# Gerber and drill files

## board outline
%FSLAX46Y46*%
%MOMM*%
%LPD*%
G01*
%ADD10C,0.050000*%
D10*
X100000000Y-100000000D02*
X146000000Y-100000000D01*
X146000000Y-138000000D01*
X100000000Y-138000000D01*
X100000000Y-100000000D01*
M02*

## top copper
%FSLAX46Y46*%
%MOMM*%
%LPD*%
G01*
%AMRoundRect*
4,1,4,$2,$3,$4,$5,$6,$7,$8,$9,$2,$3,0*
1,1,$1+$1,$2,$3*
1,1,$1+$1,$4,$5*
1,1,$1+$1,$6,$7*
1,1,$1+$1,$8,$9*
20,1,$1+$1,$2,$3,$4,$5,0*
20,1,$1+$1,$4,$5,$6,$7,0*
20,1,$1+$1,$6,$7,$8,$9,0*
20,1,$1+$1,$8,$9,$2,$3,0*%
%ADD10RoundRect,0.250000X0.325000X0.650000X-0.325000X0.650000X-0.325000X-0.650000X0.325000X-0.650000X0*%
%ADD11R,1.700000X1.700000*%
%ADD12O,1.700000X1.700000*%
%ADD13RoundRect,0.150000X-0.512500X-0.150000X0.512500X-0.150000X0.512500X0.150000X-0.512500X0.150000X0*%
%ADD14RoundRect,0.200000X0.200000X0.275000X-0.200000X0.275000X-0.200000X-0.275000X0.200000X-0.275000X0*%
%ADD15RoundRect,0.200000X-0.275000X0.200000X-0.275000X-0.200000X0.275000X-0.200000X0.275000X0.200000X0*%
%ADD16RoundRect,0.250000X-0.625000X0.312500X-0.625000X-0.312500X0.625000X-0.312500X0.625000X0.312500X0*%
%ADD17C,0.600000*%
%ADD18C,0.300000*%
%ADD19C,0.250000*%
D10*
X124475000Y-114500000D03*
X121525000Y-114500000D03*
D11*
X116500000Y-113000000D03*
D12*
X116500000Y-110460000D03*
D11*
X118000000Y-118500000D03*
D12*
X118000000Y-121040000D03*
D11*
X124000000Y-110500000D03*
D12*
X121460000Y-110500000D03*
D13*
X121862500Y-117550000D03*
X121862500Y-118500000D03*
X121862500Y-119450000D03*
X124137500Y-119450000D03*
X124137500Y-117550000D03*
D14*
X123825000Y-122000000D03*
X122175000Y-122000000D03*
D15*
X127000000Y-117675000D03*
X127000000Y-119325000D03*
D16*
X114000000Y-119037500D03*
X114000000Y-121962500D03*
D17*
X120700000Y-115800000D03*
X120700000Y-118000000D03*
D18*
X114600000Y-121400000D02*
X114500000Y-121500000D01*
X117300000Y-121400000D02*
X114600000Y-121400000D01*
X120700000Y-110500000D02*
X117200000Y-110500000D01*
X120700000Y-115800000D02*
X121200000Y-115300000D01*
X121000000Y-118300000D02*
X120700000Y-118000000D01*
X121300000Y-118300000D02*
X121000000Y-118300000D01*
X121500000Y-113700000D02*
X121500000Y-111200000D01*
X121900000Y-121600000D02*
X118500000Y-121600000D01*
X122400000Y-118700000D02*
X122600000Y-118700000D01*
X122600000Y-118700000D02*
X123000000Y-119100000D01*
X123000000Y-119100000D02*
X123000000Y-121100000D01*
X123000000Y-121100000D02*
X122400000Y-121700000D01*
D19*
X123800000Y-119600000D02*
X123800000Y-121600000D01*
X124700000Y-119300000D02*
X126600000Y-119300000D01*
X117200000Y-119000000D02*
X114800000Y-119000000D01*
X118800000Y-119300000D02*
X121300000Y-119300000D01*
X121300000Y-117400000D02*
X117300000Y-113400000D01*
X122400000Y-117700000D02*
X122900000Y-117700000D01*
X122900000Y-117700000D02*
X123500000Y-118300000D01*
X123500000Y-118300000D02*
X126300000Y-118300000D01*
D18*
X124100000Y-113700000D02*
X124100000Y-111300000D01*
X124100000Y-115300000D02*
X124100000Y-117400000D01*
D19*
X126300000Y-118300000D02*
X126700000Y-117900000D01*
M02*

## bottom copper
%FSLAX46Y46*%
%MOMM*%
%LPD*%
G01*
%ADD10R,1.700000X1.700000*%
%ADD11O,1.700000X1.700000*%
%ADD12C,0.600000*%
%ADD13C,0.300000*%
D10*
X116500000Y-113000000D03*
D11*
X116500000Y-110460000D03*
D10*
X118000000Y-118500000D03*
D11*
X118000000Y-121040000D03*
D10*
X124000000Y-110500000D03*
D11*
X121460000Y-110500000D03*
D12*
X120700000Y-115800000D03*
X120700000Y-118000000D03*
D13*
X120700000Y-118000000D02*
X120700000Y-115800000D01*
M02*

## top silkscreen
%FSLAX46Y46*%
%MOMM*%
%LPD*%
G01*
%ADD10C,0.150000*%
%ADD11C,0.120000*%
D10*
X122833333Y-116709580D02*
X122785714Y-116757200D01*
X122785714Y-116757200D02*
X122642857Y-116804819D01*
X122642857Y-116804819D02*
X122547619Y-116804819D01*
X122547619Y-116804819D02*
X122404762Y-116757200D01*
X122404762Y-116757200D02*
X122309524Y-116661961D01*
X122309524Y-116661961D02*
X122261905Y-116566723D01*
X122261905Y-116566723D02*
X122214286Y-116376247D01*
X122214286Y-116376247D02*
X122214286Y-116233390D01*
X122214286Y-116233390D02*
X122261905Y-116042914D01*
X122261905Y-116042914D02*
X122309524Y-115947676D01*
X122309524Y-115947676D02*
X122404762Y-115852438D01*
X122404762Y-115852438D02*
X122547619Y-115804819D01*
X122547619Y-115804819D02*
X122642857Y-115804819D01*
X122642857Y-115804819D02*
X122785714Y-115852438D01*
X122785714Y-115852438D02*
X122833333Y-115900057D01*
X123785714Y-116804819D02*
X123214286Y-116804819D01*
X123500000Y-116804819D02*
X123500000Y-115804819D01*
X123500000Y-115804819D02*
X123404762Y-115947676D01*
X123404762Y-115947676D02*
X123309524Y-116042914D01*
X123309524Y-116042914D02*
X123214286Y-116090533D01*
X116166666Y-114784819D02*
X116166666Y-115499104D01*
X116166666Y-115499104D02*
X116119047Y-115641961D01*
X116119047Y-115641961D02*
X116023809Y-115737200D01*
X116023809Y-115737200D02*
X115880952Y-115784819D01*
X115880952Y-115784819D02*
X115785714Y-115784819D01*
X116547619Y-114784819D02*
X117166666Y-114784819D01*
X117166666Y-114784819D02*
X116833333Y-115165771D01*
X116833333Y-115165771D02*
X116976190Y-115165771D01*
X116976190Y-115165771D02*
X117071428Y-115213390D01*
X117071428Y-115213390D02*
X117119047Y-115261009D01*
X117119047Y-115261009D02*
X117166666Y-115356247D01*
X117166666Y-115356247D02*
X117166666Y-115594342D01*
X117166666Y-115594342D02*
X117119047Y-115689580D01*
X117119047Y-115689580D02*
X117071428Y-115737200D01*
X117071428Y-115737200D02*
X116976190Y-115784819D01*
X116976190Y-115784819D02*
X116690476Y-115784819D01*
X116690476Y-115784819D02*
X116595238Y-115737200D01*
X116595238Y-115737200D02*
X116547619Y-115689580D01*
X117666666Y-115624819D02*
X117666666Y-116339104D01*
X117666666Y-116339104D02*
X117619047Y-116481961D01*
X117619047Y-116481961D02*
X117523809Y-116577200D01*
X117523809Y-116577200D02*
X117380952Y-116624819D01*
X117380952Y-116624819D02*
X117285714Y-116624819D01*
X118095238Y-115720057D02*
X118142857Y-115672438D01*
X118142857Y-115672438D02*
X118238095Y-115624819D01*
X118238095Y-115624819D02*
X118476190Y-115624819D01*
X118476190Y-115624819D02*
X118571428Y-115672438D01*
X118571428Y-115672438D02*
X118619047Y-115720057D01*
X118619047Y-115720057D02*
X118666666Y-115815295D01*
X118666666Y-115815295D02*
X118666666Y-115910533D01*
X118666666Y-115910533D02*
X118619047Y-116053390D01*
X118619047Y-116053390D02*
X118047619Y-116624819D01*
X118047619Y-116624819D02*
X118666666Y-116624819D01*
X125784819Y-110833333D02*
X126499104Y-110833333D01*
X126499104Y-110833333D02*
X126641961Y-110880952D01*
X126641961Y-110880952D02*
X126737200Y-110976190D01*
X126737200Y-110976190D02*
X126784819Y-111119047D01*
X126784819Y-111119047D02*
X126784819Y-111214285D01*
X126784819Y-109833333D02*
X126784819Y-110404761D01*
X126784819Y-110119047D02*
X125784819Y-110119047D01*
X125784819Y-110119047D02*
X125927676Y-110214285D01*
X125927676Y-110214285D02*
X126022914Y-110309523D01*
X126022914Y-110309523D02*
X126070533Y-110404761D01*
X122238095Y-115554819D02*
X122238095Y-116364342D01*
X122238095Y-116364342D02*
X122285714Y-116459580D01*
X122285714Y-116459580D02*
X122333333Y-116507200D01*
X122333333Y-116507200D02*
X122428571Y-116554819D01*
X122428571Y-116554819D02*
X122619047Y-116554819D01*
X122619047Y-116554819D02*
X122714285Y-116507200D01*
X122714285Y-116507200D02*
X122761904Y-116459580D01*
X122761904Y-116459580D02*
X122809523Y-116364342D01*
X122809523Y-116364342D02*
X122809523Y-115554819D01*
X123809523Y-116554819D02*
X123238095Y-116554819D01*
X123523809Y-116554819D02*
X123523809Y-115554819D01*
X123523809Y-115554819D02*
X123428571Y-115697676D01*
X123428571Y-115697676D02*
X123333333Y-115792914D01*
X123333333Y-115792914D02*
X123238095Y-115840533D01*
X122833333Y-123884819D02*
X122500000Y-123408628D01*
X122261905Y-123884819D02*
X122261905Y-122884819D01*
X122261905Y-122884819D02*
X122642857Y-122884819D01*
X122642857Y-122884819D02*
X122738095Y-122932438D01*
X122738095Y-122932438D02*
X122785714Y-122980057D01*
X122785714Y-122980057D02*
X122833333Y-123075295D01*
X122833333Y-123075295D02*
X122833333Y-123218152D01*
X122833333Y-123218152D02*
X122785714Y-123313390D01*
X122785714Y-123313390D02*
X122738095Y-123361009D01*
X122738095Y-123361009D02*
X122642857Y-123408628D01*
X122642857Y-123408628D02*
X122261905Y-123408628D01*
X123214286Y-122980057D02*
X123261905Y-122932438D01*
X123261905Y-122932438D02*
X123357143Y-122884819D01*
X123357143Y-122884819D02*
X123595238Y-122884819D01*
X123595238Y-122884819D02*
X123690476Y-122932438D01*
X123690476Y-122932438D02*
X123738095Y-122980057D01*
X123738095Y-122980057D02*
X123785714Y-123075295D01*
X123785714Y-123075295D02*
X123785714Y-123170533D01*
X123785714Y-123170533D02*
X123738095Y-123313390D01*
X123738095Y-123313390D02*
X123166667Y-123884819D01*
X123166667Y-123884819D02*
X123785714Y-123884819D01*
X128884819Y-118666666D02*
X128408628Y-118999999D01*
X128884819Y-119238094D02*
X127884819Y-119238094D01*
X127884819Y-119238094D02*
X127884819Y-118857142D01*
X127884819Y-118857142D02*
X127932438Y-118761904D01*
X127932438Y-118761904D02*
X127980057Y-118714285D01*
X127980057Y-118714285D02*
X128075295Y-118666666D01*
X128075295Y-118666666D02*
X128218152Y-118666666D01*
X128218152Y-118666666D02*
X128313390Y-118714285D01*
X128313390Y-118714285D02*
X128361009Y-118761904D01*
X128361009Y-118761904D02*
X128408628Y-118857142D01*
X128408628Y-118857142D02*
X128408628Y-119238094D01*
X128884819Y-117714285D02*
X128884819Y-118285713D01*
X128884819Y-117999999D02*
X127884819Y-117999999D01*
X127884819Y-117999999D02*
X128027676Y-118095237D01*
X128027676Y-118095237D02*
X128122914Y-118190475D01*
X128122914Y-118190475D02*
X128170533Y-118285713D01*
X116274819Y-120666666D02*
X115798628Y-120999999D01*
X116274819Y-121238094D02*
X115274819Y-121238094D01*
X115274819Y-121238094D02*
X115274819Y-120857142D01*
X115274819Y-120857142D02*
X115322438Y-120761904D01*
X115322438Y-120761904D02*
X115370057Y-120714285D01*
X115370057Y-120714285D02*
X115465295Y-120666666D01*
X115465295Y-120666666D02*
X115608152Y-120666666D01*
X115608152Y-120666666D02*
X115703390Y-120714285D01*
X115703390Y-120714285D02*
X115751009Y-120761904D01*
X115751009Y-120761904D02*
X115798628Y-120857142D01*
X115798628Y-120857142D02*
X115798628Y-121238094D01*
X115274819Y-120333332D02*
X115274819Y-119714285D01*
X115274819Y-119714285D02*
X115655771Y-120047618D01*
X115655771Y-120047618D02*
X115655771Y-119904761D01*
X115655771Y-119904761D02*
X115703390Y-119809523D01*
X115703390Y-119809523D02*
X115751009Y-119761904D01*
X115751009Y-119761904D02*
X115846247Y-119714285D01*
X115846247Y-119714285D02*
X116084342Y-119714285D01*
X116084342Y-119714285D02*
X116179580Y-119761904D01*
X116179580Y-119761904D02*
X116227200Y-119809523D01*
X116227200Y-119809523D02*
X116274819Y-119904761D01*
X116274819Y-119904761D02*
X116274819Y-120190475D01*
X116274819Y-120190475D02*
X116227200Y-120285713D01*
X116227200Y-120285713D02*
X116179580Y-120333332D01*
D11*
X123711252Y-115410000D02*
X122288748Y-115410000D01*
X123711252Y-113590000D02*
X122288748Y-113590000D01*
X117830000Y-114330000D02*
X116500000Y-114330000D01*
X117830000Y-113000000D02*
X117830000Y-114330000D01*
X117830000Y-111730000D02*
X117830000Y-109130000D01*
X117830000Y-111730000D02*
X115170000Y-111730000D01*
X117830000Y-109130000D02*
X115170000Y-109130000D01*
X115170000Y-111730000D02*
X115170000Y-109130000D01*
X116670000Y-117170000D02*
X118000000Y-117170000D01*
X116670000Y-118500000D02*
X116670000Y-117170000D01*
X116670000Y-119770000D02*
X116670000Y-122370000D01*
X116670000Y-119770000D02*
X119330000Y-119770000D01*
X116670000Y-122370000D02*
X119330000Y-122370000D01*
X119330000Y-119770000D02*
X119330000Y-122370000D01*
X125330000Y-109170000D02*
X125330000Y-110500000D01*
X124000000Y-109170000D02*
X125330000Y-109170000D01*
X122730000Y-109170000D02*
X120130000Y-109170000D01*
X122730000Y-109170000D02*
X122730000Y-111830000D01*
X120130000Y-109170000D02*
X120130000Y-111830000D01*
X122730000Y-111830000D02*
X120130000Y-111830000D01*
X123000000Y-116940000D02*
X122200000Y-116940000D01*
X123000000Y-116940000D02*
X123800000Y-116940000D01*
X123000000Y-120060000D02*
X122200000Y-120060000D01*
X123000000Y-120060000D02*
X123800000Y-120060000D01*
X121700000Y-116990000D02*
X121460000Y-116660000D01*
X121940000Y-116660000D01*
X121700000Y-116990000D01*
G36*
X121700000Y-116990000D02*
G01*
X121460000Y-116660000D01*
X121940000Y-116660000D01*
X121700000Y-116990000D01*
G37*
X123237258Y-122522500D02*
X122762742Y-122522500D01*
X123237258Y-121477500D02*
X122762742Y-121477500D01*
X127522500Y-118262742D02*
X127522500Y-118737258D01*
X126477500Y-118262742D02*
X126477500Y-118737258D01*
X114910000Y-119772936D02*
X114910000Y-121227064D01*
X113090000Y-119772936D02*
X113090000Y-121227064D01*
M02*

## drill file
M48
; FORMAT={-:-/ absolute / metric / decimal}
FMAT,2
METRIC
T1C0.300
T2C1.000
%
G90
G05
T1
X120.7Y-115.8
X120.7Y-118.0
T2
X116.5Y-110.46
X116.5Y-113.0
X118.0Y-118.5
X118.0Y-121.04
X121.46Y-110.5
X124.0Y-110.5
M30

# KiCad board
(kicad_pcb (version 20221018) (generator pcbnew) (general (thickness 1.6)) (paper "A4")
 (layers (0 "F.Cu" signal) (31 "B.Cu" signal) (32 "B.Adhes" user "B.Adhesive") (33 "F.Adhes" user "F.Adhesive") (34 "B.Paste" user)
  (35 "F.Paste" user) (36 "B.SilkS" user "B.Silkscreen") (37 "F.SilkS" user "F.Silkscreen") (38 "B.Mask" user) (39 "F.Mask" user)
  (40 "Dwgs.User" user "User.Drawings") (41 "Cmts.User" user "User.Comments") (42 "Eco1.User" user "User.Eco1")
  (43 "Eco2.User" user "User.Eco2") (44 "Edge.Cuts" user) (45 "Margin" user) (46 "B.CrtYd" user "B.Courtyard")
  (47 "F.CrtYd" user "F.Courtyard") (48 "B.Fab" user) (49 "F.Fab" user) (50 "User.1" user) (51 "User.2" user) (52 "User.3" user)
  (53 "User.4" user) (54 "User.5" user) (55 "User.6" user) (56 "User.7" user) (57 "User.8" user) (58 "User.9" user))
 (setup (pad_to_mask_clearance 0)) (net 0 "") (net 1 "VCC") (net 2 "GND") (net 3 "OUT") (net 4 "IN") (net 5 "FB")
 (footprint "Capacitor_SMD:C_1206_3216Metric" (layer "F.Cu") (at 123 114.5 180)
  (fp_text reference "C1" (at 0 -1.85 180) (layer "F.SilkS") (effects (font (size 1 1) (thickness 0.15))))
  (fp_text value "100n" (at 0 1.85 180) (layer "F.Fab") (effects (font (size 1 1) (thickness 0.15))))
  (fp_line (start -0.711252 -0.91) (end 0.711252 -0.91) (stroke (width 0.12) (type solid)) (layer "F.SilkS"))
  (fp_line (start -0.711252 0.91) (end 0.711252 0.91) (stroke (width 0.12) (type solid)) (layer "F.SilkS"))
  (pad "1" smd roundrect (at -1.475 0 180) (size 1.15 1.8) (layers "F.Cu" "F.Paste" "F.Mask") (roundrect_rratio 0.217391) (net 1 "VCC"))
  (pad "2" smd roundrect (at 1.475 0 180) (size 1.15 1.8) (layers "F.Cu" "F.Paste" "F.Mask") (roundrect_rratio 0.217391) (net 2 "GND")))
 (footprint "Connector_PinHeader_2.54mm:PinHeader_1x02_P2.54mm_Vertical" (layer "F.Cu") (at 116.5 113 180)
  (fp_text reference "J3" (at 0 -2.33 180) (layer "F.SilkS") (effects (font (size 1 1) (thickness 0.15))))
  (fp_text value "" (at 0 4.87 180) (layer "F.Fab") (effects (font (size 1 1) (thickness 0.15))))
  (fp_line (start -1.33 -1.33) (end 0 -1.33) (stroke (width 0.12) (type solid)) (layer "F.SilkS"))
  (fp_line (start -1.33 0) (end -1.33 -1.33) (stroke (width 0.12) (type solid)) (layer "F.SilkS"))
  (fp_line (start -1.33 1.27) (end -1.33 3.87) (stroke (width 0.12) (type solid)) (layer "F.SilkS"))
  (fp_line (start -1.33 1.27) (end 1.33 1.27) (stroke (width 0.12) (type solid)) (layer "F.SilkS"))
  (fp_line (start -1.33 3.87) (end 1.33 3.87) (stroke (width 0.12) (type solid)) (layer "F.SilkS"))
  (fp_line (start 1.33 1.27) (end 1.33 3.87) (stroke (width 0.12) (type solid)) (layer "F.SilkS"))
  (pad "1" thru_hole rect (at 0 0 180) (size 1.7 1.7) (drill 1) (layers "*.Cu" "*.Mask") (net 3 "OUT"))
  (pad "2" thru_hole oval (at 0 2.54 180) (size 1.7 1.7) (drill 1) (layers "*.Cu" "*.Mask") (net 2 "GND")))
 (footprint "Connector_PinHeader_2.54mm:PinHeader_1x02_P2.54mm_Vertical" (layer "F.Cu") (at 118 118.5)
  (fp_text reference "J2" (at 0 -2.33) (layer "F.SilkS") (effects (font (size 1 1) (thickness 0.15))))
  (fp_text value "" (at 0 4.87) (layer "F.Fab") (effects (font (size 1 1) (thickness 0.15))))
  (fp_line (start -1.33 -1.33) (end 0 -1.33) (stroke (width 0.12) (type solid)) (layer "F.SilkS"))
  (fp_line (start -1.33 0) (end -1.33 -1.33) (stroke (width 0.12) (type solid)) (layer "F.SilkS"))
  (fp_line (start -1.33 1.27) (end -1.33 3.87) (stroke (width 0.12) (type solid)) (layer "F.SilkS"))
  (fp_line (start -1.33 1.27) (end 1.33 1.27) (stroke (width 0.12) (type solid)) (layer "F.SilkS"))
  (fp_line (start -1.33 3.87) (end 1.33 3.87) (stroke (width 0.12) (type solid)) (layer "F.SilkS"))
  (fp_line (start 1.33 1.27) (end 1.33 3.87) (stroke (width 0.12) (type solid)) (layer "F.SilkS"))
  (pad "1" thru_hole rect (at 0 0) (size 1.7 1.7) (drill 1) (layers "*.Cu" "*.Mask") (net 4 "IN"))
  (pad "2" thru_hole oval (at 0 2.54) (size 1.7 1.7) (drill 1) (layers "*.Cu" "*.Mask") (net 2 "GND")))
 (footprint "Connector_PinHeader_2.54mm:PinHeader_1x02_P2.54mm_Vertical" (layer "F.Cu") (at 124 110.5 -90)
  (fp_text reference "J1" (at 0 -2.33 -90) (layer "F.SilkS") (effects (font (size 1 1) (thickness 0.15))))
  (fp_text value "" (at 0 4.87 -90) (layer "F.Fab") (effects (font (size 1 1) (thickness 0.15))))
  (fp_line (start -1.33 -1.33) (end 0 -1.33) (stroke (width 0.12) (type solid)) (layer "F.SilkS"))
  (fp_line (start -1.33 0) (end -1.33 -1.33) (stroke (width 0.12) (type solid)) (layer "F.SilkS"))
  (fp_line (start -1.33 1.27) (end -1.33 3.87) (stroke (width 0.12) (type solid)) (layer "F.SilkS"))
  (fp_line (start -1.33 1.27) (end 1.33 1.27) (stroke (width 0.12) (type solid)) (layer "F.SilkS"))
  (fp_line (start -1.33 3.87) (end 1.33 3.87) (stroke (width 0.12) (type solid)) (layer "F.SilkS"))
  (fp_line (start 1.33 1.27) (end 1.33 3.87) (stroke (width 0.12) (type solid)) (layer "F.SilkS"))
  (pad "1" thru_hole rect (at 0 0 270) (size 1.7 1.7) (drill 1) (layers "*.Cu" "*.Mask") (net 1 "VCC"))
  (pad "2" thru_hole oval (at 0 2.54 270) (size 1.7 1.7) (drill 1) (layers "*.Cu" "*.Mask") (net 2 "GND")))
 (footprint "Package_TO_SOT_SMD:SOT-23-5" (layer "F.Cu") (at 123 118.5)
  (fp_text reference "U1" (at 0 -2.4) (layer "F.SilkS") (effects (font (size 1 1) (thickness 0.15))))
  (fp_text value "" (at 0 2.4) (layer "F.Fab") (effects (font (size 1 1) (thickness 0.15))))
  (fp_line (start 0 -1.56) (end -0.8 -1.56) (stroke (width 0.12) (type solid)) (layer "F.SilkS"))
  (fp_line (start 0 -1.56) (end 0.8 -1.56) (stroke (width 0.12) (type solid)) (layer "F.SilkS"))
  (fp_line (start 0 1.56) (end -0.8 1.56) (stroke (width 0.12) (type solid)) (layer "F.SilkS"))
  (fp_line (start 0 1.56) (end 0.8 1.56) (stroke (width 0.12) (type solid)) (layer "F.SilkS"))
  (fp_poly
   (pts (xy -1.3 -1.51) (xy -1.54 -1.84) (xy -1.06 -1.84) (xy -1.3 -1.51)) (stroke (width 0.12) (type solid)) (fill solid) (layer "F.SilkS"))
  (pad "1" smd roundrect (at -1.1375 -0.95) (size 1.325 0.6) (layers "F.Cu" "F.Paste" "F.Mask") (roundrect_rratio 0.25) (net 3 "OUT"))
  (pad "2" smd roundrect (at -1.1375 0) (size 1.325 0.6) (layers "F.Cu" "F.Paste" "F.Mask") (roundrect_rratio 0.25) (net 2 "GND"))
  (pad "3" smd roundrect (at -1.1375 0.95) (size 1.325 0.6) (layers "F.Cu" "F.Paste" "F.Mask") (roundrect_rratio 0.25) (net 4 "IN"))
  (pad "4" smd roundrect (at 1.1375 0.95) (size 1.325 0.6) (layers "F.Cu" "F.Paste" "F.Mask") (roundrect_rratio 0.25) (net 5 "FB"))
  (pad "5" smd roundrect (at 1.1375 -0.95) (size 1.325 0.6) (layers "F.Cu" "F.Paste" "F.Mask") (roundrect_rratio 0.25) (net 1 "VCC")))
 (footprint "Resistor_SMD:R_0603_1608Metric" (layer "F.Cu") (at 123 122 180)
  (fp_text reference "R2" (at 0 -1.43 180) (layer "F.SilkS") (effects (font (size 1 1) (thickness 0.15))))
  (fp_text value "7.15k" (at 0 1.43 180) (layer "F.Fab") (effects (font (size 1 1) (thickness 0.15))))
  (fp_line (start -0.237258 -0.5225) (end 0.237258 -0.5225) (stroke (width 0.12) (type solid)) (layer "F.SilkS"))
  (fp_line (start -0.237258 0.5225) (end 0.237258 0.5225) (stroke (width 0.12) (type solid)) (layer "F.SilkS"))
  (pad "1" smd roundrect (at -0.825 0 180) (size 0.8 0.95) (layers "F.Cu" "F.Paste" "F.Mask") (roundrect_rratio 0.25) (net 5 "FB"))
  (pad "2" smd roundrect (at 0.825 0 180) (size 0.8 0.95) (layers "F.Cu" "F.Paste" "F.Mask") (roundrect_rratio 0.25) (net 2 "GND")))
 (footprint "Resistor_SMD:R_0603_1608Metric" (layer "F.Cu") (at 127 118.5 -90)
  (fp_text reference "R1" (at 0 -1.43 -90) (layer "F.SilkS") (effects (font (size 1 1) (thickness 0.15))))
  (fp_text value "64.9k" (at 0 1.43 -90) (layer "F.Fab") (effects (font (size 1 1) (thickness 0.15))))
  (fp_line (start -0.237258 -0.5225) (end 0.237258 -0.5225) (stroke (width 0.12) (type solid)) (layer "F.SilkS"))
  (fp_line (start -0.237258 0.5225) (end 0.237258 0.5225) (stroke (width 0.12) (type solid)) (layer "F.SilkS"))
  (pad "1" smd roundrect (at -0.825 0 270) (size 0.8 0.95) (layers "F.Cu" "F.Paste" "F.Mask") (roundrect_rratio 0.25) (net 3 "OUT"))
  (pad "2" smd roundrect (at 0.825 0 270) (size 0.8 0.95) (layers "F.Cu" "F.Paste" "F.Mask") (roundrect_rratio 0.25) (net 5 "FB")))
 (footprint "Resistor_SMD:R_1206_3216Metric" (layer "F.Cu") (at 114 120.5 -90)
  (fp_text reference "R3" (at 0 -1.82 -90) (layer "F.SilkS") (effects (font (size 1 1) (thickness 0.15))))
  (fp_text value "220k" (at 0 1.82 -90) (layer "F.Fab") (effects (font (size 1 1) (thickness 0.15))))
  (fp_line (start -0.727064 -0.91) (end 0.727064 -0.91) (stroke (width 0.12) (type solid)) (layer "F.SilkS"))
  (fp_line (start -0.727064 0.91) (end 0.727064 0.91) (stroke (width 0.12) (type solid)) (layer "F.SilkS"))
  (pad "1" smd roundrect (at -1.4625 0 270) (size 1.125 1.75) (layers "F.Cu" "F.Paste" "F.Mask") (roundrect_rratio 0.222222) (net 4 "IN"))
  (pad "2" smd roundrect (at 1.4625 0 270) (size 1.125 1.75) (layers "F.Cu" "F.Paste" "F.Mask") (roundrect_rratio 0.222222) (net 2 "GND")))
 (gr_rect (start 100 100) (end 146 138) (stroke (width 0.05) (type default)) (fill none) (layer "Edge.Cuts"))
 (segment (start 114.6 121.4) (end 114.5 121.5) (width 0.3) (layer "F.Cu") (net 2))
 (segment (start 117.3 121.4) (end 114.6 121.4) (width 0.3) (layer "F.Cu") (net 2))
 (segment (start 120.7 110.5) (end 117.2 110.5) (width 0.3) (layer "F.Cu") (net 2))
 (segment (start 120.7 115.8) (end 121.2 115.3) (width 0.3) (layer "F.Cu") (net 2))
 (segment (start 121 118.3) (end 120.7 118) (width 0.3) (layer "F.Cu") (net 2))
 (segment (start 121.3 118.3) (end 121 118.3) (width 0.3) (layer "F.Cu") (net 2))
 (segment (start 121.5 113.7) (end 121.5 111.2) (width 0.3) (layer "F.Cu") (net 2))
 (segment (start 121.9 121.6) (end 118.5 121.6) (width 0.3) (layer "F.Cu") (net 2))
 (segment (start 122.4 118.7) (end 122.6 118.7) (width 0.3) (layer "F.Cu") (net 2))
 (segment (start 122.6 118.7) (end 123 119.1) (width 0.3) (layer "F.Cu") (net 2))
 (segment (start 123 119.1) (end 123 121.1) (width 0.3) (layer "F.Cu") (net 2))
 (segment (start 123 121.1) (end 122.4 121.7) (width 0.3) (layer "F.Cu") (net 2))
 (segment (start 123.8 119.6) (end 123.8 121.6) (width 0.25) (layer "F.Cu") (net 5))
 (segment (start 124.7 119.3) (end 126.6 119.3) (width 0.25) (layer "F.Cu") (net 5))
 (via (at 120.7 115.8) (size 0.6) (drill 0.3) (layers "F.Cu" "B.Cu") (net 2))
 (via (at 120.7 118) (size 0.6) (drill 0.3) (layers "F.Cu" "B.Cu") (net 2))
 (segment (start 117.2 119) (end 114.8 119) (width 0.25) (layer "F.Cu") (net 4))
 (segment (start 118.8 119.3) (end 121.3 119.3) (width 0.25) (layer "F.Cu") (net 4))
 (segment (start 120.7 118) (end 120.7 115.8) (width 0.3) (layer "B.Cu") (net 2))
 (segment (start 121.3 117.4) (end 117.3 113.4) (width 0.25) (layer "F.Cu") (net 3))
 (segment (start 122.4 117.7) (end 122.9 117.7) (width 0.25) (layer "F.Cu") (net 3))
 (segment (start 122.9 117.7) (end 123.5 118.3) (width 0.25) (layer "F.Cu") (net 3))
 (segment (start 123.5 118.3) (end 126.3 118.3) (width 0.25) (layer "F.Cu") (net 3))
 (segment (start 124.1 113.7) (end 124.1 111.3) (width 0.3) (layer "F.Cu") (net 1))
 (segment (start 124.1 115.3) (end 124.1 117.4) (width 0.3) (layer "F.Cu") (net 1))
 (segment (start 126.3 118.3) (end 126.7 117.9) (width 0.25) (layer "F.Cu") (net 3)))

